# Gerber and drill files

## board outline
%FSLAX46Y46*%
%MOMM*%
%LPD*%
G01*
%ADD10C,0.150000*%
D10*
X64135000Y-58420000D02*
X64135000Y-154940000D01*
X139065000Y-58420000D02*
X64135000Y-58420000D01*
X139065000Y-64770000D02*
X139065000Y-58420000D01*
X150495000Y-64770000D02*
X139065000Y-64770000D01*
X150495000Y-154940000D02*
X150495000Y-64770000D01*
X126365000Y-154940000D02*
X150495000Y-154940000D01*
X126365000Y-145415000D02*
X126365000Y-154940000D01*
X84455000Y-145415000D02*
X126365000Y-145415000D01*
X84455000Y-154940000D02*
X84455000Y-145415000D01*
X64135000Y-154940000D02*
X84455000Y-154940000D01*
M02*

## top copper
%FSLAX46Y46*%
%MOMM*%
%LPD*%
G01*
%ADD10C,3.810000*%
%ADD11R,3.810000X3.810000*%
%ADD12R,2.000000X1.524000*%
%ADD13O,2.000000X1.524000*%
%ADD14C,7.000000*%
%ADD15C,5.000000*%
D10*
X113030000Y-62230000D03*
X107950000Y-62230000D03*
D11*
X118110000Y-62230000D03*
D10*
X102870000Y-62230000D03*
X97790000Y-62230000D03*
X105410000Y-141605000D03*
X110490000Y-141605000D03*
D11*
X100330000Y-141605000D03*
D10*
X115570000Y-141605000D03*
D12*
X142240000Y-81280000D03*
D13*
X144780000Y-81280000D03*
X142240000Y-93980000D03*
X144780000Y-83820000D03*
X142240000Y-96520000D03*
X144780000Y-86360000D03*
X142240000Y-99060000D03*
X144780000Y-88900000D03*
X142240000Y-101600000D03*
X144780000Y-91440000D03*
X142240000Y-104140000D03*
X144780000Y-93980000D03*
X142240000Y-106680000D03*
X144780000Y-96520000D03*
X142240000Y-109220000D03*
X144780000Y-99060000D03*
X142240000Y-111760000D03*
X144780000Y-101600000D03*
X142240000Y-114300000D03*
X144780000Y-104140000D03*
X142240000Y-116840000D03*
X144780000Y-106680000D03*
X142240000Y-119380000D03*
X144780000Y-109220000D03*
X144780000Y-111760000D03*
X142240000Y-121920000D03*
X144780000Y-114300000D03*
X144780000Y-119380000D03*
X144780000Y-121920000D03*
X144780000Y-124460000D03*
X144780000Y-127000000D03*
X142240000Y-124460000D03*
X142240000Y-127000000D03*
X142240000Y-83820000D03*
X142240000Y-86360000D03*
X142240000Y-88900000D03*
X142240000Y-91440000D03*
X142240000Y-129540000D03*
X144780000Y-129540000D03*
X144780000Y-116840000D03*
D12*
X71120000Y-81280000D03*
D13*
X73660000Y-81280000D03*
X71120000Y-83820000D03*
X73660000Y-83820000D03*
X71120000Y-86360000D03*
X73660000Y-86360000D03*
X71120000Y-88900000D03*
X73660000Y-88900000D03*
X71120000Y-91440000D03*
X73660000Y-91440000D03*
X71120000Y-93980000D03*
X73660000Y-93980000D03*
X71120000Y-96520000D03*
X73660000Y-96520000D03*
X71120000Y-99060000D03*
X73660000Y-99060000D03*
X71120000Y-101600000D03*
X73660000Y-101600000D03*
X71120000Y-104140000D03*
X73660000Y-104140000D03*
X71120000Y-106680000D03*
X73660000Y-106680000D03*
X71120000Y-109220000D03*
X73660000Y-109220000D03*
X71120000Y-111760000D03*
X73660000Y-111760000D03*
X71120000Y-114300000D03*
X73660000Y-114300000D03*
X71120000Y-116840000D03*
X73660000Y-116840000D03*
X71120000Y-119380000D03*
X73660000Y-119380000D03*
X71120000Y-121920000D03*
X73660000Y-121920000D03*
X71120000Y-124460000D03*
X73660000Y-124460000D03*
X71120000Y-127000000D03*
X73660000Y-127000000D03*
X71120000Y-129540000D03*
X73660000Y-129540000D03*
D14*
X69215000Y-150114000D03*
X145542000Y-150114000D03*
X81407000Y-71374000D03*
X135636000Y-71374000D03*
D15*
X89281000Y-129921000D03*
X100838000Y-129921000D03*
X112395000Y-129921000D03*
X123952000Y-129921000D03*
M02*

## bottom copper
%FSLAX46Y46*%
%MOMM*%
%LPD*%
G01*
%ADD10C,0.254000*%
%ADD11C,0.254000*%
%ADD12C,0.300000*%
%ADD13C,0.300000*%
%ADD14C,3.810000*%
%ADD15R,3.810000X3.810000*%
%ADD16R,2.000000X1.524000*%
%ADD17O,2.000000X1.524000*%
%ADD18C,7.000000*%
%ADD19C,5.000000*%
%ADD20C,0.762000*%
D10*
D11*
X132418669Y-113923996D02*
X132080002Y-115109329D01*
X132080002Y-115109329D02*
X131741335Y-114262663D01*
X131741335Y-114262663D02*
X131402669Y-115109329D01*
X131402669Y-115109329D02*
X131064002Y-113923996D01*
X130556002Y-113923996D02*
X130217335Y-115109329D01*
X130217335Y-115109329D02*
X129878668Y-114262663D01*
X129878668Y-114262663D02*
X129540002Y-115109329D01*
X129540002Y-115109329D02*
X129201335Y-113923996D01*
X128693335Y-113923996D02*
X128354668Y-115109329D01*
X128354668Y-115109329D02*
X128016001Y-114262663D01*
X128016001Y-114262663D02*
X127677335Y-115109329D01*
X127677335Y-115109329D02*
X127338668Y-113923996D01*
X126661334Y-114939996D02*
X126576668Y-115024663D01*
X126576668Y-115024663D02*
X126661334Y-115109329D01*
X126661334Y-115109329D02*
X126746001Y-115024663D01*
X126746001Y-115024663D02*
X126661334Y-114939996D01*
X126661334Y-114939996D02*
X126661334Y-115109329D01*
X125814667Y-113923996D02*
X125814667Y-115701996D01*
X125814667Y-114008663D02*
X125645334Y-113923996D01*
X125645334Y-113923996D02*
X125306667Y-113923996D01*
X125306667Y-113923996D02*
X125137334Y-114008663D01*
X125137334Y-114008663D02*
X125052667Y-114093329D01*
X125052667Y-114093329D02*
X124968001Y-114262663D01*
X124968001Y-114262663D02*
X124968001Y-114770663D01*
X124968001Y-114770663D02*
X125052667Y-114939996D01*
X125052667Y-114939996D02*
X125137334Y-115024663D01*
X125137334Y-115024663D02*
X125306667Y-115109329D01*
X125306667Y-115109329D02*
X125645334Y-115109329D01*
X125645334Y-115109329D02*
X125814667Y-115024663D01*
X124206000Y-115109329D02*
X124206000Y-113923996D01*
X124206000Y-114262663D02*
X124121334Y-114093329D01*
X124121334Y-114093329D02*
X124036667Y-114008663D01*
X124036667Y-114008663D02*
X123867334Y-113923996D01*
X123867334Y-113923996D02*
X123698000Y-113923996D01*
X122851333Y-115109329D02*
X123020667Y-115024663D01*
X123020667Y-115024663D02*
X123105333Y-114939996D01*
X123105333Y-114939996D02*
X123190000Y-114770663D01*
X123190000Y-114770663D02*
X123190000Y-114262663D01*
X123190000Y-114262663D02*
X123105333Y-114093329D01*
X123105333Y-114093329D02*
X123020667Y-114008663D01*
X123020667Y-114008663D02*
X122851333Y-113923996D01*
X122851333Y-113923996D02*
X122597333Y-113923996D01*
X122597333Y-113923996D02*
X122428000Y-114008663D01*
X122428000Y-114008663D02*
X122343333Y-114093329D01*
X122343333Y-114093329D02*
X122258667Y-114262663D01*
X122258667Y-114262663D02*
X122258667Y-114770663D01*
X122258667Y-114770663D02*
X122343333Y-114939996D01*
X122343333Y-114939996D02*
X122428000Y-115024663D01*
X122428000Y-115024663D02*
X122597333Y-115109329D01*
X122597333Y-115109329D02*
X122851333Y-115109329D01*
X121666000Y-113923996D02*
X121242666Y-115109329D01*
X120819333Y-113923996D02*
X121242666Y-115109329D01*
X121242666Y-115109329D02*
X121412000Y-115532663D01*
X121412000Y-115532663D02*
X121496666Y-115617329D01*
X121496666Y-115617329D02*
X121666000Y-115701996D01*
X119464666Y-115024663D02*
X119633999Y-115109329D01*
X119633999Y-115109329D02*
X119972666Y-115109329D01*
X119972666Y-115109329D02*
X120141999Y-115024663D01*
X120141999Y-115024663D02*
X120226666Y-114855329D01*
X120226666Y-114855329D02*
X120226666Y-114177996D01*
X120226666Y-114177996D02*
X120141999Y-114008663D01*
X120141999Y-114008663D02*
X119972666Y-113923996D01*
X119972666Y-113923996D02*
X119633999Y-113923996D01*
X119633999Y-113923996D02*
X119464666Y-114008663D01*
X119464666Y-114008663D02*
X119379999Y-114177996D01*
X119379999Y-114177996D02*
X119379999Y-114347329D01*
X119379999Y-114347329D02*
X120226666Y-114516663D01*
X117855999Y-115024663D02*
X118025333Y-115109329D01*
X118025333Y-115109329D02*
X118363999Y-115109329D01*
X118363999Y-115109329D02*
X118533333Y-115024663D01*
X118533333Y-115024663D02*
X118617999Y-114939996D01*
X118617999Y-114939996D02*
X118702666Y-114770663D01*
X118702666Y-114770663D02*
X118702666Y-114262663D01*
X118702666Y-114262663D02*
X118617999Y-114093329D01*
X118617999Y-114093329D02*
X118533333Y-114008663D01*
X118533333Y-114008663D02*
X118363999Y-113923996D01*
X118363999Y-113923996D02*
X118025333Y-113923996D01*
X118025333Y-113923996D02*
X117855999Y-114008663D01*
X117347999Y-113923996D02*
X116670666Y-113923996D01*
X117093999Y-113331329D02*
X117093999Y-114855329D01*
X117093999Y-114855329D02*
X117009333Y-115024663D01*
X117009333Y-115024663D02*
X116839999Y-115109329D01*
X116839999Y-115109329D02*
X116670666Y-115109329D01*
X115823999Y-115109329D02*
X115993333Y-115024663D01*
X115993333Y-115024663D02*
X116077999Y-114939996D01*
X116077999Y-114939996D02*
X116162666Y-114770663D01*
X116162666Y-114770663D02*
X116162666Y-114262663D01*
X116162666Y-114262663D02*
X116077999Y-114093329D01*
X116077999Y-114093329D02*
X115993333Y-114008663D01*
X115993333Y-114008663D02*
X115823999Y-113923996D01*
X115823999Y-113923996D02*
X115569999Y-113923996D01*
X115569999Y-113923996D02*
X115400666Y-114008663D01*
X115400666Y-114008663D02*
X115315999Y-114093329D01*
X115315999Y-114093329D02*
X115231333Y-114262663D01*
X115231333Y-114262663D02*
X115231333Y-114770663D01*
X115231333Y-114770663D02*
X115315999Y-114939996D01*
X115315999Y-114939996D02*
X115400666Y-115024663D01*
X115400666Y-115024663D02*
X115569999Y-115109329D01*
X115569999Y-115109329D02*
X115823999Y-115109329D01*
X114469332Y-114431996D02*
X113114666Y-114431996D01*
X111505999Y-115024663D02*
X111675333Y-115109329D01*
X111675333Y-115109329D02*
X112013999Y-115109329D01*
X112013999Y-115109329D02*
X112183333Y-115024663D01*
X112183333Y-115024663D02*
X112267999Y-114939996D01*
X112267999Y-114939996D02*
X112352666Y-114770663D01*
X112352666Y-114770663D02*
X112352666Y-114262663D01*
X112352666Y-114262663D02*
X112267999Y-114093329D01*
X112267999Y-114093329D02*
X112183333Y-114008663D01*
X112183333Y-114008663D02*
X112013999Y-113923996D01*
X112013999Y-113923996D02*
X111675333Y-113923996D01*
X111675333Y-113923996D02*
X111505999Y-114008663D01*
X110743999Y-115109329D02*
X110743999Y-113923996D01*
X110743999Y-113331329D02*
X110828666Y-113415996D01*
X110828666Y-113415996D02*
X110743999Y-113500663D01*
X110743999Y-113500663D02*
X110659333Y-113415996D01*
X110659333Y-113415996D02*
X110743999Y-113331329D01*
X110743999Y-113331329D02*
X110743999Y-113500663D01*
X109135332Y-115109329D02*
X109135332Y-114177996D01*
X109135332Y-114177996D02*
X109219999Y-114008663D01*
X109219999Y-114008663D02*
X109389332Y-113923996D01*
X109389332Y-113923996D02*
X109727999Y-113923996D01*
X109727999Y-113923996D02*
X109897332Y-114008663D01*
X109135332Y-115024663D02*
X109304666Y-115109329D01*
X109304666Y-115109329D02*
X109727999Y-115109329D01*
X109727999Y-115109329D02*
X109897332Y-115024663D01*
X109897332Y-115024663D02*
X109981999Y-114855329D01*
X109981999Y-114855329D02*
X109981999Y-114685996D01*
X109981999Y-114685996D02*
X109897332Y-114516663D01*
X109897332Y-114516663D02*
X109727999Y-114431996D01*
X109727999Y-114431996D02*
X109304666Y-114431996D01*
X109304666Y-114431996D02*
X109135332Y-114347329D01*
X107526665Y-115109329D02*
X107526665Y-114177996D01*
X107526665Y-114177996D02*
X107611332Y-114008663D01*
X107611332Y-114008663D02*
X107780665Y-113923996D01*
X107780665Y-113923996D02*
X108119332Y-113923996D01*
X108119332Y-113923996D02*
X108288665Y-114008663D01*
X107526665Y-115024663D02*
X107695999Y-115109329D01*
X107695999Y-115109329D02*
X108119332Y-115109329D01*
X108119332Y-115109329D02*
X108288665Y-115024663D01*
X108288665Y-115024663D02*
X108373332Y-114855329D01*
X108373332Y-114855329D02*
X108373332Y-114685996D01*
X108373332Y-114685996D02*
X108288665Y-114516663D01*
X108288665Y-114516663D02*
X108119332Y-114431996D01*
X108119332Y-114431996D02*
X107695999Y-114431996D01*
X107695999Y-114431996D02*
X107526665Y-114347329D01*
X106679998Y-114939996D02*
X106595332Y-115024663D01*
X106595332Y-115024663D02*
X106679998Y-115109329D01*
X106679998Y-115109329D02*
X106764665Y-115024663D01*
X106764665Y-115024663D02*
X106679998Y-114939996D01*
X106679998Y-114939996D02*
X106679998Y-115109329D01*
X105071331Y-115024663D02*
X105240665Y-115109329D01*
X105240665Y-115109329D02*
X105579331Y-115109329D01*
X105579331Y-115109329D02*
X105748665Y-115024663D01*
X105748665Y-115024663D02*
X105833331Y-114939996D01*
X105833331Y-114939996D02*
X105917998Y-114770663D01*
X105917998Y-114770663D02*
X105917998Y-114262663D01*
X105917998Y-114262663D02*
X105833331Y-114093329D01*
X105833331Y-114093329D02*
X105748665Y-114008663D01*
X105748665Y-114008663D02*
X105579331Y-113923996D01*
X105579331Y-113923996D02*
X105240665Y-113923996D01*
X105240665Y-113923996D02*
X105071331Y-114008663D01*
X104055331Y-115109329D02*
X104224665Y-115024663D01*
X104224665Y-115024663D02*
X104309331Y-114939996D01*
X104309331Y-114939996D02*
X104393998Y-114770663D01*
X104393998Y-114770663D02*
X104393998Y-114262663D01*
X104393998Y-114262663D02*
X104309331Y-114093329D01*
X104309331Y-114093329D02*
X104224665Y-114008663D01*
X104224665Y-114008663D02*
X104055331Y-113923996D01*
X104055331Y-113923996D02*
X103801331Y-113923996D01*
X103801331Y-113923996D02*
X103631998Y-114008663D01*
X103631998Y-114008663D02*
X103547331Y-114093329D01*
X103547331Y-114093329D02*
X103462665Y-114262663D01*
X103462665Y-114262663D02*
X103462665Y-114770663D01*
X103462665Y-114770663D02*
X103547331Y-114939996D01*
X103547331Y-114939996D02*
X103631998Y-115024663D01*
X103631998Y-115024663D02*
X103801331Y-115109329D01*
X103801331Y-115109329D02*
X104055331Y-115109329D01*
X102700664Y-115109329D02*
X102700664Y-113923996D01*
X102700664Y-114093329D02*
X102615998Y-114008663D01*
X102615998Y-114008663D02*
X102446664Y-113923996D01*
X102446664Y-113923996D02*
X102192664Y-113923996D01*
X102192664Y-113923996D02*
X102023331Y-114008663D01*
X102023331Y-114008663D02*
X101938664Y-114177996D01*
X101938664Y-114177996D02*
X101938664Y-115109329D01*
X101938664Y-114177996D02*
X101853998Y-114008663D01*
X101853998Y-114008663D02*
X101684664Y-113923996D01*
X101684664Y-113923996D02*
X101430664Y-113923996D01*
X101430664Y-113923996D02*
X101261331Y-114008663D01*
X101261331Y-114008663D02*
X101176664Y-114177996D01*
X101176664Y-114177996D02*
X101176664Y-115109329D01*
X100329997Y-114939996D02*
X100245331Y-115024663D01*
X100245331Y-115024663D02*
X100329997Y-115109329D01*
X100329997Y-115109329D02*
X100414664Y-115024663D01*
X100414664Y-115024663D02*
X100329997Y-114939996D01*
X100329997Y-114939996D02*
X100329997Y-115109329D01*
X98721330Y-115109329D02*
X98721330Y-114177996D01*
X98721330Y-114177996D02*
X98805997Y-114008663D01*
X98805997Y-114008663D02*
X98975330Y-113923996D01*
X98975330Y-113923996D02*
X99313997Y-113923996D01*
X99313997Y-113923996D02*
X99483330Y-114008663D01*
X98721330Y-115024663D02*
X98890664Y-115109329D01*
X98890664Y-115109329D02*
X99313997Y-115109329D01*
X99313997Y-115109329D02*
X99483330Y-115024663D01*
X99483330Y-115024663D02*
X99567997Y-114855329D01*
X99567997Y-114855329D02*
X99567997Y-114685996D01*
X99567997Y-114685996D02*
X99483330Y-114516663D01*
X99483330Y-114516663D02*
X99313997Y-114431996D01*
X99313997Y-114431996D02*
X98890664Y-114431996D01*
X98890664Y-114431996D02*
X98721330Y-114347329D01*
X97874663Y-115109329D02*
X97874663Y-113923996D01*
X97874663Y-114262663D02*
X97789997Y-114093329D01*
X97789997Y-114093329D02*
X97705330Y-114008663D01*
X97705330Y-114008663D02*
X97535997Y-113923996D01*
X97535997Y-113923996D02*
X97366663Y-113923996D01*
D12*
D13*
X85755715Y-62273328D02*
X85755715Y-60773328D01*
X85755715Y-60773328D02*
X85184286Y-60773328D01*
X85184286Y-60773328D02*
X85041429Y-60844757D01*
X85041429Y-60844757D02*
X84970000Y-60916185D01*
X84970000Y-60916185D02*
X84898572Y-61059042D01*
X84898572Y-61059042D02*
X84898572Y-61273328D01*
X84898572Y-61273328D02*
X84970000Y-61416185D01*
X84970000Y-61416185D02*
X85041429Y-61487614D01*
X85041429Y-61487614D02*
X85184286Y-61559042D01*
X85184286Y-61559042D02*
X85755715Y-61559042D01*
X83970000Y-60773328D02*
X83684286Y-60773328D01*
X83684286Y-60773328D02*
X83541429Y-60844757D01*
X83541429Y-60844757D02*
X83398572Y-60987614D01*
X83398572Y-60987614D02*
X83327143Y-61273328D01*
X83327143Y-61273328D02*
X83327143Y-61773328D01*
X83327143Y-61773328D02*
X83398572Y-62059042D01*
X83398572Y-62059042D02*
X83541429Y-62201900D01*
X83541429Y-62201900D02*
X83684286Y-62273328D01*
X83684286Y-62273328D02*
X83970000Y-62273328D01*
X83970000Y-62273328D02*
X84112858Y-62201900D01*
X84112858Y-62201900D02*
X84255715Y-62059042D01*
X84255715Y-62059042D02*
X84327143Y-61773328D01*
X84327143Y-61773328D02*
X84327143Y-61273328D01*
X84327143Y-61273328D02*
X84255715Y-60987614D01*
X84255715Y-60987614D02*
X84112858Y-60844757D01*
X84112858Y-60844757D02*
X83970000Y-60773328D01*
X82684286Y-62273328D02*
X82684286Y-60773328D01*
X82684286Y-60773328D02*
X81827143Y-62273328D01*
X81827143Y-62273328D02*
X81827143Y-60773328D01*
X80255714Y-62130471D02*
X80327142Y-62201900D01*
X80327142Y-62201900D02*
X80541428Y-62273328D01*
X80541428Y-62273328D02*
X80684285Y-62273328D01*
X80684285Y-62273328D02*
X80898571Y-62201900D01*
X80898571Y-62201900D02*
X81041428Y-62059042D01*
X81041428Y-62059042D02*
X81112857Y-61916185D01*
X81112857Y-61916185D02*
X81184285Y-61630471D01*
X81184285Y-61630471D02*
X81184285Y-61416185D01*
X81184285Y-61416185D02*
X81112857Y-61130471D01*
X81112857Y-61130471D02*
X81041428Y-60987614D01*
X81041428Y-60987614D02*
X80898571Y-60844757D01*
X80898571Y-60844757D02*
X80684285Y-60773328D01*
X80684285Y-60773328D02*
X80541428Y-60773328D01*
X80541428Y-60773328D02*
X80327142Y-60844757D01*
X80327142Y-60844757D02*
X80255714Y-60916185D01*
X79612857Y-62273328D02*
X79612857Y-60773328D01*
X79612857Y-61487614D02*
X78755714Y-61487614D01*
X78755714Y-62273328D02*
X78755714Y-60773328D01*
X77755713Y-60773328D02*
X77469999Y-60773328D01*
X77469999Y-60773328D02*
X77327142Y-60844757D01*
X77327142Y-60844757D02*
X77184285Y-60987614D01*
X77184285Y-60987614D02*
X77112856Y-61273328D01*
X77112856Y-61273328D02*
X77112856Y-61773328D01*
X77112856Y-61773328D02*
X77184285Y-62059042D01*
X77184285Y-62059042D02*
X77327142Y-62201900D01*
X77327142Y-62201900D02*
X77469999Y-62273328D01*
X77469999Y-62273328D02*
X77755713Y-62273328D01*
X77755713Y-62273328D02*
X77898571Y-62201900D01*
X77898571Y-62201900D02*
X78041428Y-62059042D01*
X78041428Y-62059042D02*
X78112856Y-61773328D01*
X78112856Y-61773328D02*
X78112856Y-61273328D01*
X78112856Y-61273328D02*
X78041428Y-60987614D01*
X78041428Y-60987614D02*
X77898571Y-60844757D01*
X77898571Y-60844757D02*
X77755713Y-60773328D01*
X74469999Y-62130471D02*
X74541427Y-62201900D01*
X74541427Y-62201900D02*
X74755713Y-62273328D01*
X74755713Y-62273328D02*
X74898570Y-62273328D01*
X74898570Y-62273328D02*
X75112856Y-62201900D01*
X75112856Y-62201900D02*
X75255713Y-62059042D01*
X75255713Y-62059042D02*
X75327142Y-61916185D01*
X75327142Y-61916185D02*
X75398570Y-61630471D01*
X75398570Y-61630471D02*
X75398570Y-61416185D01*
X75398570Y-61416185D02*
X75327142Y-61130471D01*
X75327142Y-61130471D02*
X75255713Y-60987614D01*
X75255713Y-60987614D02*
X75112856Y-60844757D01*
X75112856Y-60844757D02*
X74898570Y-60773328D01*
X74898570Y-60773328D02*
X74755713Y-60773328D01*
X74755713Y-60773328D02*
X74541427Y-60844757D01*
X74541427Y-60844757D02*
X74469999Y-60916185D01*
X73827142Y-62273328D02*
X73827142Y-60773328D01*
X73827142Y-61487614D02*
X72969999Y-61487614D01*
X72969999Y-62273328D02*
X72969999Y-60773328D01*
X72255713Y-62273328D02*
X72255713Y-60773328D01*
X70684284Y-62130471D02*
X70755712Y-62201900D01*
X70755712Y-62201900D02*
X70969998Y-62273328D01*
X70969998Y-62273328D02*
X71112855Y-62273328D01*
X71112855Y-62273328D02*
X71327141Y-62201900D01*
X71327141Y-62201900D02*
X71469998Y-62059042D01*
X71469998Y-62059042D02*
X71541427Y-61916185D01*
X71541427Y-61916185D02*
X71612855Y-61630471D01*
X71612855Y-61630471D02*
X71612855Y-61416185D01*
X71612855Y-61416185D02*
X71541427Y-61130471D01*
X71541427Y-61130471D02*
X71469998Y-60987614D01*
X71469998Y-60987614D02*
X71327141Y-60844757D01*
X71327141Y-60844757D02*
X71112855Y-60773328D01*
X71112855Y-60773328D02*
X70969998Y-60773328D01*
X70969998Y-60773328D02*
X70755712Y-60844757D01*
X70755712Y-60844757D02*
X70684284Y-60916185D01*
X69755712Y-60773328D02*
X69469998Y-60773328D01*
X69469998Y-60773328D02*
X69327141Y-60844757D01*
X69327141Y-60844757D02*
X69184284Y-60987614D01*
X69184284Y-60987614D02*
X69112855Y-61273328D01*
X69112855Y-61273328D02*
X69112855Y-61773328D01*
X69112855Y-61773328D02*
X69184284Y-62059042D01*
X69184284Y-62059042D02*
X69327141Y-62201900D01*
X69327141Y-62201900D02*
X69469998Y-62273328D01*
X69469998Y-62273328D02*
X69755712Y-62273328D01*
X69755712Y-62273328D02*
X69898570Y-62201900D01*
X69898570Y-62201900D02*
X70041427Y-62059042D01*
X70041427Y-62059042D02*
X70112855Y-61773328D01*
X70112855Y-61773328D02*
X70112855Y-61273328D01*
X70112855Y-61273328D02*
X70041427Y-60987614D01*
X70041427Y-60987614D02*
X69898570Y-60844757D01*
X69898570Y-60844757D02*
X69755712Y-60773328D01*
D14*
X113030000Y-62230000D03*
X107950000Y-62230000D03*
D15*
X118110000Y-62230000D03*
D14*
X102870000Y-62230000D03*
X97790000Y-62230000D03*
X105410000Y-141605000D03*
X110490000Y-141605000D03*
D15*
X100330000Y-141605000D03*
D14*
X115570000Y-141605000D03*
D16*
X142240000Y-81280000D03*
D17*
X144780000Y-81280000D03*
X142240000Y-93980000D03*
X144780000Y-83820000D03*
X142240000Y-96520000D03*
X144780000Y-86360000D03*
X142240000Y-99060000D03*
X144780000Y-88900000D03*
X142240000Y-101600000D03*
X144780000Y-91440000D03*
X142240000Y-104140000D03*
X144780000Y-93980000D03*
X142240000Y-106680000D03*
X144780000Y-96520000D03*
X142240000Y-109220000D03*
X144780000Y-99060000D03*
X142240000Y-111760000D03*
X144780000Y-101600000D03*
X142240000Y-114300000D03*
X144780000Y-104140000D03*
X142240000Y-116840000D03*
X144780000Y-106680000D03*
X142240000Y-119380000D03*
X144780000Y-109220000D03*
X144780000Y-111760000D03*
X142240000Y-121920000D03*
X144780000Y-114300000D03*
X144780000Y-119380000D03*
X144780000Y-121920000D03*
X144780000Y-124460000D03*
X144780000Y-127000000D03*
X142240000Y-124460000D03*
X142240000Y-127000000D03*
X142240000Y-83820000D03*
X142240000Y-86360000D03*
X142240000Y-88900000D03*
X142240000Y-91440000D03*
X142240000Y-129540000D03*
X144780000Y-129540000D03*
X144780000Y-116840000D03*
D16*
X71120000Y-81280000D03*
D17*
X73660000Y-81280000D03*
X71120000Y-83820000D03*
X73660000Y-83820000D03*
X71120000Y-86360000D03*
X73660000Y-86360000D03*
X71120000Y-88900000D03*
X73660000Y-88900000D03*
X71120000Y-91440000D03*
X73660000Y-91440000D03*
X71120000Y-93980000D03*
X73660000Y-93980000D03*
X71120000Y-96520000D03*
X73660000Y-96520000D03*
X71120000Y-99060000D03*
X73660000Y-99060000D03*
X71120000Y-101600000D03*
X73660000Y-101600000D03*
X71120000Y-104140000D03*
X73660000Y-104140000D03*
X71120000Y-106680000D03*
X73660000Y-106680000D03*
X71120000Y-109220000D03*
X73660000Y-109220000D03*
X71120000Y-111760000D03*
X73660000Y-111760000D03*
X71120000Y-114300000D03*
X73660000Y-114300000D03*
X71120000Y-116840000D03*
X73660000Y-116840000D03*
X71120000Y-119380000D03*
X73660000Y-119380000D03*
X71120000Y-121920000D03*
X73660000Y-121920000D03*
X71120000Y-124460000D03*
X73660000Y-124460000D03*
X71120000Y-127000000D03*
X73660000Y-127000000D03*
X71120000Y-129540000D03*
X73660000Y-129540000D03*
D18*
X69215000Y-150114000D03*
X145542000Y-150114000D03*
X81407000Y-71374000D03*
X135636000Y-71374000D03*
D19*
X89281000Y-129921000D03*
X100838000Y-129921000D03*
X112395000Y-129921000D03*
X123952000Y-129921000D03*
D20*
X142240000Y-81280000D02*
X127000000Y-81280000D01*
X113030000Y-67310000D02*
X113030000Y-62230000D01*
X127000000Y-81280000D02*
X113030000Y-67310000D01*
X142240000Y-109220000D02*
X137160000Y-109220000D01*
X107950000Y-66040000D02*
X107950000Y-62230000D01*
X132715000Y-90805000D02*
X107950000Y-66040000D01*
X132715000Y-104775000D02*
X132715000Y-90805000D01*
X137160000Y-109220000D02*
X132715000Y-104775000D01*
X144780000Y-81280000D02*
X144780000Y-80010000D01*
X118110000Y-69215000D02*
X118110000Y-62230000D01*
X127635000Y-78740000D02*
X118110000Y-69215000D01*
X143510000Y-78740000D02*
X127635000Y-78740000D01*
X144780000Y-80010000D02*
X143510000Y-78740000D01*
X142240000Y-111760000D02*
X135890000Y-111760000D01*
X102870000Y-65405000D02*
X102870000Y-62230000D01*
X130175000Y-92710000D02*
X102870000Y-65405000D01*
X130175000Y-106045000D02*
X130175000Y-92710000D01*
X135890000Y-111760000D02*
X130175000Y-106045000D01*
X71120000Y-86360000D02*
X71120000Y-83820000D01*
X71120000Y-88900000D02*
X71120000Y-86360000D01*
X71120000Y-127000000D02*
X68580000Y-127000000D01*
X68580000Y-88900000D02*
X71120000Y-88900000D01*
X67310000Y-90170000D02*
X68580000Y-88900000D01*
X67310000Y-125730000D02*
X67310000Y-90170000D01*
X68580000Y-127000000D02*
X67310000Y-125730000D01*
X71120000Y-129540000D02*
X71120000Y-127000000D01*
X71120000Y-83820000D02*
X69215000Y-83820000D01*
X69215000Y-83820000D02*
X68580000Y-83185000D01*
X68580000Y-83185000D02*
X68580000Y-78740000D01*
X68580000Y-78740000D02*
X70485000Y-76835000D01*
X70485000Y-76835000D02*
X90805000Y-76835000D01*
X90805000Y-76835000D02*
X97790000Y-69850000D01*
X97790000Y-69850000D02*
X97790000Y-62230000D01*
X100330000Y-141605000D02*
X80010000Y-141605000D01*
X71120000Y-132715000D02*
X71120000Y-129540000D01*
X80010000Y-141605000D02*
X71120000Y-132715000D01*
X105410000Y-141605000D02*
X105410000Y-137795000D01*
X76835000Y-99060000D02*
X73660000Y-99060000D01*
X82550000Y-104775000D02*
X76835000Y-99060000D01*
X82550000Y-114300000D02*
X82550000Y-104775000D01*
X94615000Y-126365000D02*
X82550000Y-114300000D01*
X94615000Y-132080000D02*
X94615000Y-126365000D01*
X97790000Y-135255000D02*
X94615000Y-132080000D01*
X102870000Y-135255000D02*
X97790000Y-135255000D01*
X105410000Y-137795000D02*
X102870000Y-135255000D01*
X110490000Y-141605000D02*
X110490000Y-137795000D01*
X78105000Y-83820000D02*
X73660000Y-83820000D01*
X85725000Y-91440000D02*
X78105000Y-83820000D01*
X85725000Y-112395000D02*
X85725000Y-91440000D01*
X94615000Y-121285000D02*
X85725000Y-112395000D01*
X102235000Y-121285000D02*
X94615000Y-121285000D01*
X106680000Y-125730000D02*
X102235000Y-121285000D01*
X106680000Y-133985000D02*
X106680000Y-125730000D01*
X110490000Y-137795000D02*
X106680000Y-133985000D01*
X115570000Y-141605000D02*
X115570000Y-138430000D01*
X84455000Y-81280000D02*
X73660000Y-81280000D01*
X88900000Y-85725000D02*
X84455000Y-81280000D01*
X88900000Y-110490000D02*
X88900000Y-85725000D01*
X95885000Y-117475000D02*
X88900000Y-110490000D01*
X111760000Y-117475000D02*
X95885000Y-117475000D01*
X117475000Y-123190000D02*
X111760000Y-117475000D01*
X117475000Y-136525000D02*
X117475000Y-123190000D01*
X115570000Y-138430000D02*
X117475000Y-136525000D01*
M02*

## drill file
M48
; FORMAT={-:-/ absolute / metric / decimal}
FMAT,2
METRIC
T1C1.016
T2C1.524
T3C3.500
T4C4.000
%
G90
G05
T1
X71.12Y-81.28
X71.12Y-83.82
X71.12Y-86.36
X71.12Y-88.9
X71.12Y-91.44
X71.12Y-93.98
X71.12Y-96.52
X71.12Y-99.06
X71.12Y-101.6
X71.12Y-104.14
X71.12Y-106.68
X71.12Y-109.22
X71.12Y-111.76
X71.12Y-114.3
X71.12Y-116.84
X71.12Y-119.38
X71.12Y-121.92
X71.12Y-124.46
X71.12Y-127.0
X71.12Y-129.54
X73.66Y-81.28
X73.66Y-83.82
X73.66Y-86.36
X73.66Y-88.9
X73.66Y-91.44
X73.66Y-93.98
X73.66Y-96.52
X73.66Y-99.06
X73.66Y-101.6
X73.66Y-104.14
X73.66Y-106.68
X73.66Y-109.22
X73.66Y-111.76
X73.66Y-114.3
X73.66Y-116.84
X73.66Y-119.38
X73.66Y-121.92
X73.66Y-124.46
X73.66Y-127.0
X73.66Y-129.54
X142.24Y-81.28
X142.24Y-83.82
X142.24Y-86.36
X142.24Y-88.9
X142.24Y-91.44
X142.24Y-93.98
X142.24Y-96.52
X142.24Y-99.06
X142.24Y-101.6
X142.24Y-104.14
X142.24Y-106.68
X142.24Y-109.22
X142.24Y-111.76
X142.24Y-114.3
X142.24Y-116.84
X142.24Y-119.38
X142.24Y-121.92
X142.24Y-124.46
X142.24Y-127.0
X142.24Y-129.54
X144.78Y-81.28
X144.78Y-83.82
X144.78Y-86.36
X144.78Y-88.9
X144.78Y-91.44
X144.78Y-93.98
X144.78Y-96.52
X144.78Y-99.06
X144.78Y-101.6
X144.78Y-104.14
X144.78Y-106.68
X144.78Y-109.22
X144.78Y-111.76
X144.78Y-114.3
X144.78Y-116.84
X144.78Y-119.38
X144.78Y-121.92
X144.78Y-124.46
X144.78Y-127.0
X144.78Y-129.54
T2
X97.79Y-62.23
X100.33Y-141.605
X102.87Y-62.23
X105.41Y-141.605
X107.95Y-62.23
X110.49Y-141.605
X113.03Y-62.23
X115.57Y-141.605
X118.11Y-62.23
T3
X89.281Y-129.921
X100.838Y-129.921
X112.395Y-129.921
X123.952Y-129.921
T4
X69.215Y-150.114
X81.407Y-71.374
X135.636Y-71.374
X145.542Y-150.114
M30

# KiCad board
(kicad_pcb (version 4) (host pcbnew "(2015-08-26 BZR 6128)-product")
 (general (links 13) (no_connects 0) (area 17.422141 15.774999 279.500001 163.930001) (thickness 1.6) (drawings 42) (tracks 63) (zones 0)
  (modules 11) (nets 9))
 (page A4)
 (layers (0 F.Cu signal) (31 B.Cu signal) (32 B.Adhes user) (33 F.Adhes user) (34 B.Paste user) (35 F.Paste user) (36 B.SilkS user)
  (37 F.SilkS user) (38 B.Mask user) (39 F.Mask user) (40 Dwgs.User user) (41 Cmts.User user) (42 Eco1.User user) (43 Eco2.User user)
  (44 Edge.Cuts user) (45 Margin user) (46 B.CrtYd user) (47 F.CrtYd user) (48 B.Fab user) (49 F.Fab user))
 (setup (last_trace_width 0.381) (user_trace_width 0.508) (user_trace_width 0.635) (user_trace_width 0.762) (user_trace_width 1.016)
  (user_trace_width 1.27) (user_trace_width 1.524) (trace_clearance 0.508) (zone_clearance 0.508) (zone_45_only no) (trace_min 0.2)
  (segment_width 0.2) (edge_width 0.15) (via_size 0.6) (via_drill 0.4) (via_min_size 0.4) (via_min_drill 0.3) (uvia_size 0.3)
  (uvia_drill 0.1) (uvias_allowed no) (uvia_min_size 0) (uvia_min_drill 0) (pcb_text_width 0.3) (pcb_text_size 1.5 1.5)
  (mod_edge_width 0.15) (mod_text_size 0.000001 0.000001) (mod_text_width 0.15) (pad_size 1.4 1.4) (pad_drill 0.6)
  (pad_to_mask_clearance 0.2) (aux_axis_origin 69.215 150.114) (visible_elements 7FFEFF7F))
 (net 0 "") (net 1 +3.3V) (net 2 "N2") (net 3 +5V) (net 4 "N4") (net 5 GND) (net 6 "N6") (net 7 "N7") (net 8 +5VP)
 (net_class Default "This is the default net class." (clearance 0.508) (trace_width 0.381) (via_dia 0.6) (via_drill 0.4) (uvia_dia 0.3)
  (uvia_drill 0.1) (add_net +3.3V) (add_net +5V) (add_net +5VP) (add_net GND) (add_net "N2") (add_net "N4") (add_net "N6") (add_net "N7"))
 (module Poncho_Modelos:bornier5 (layer F.Cu) (at 107.95 62.23 180)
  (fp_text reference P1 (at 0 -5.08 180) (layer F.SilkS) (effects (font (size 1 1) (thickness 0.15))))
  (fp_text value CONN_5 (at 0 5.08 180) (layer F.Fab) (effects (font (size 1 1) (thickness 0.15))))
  (pad 2 thru_hole circle (at -5.08 0 180) (size 3.81 3.81) (drill 1.524) (layers *.Cu *.Mask F.SilkS) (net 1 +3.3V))
  (pad 3 thru_hole circle (at 0 0 180) (size 3.81 3.81) (drill 1.524) (layers *.Cu *.Mask F.SilkS) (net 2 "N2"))
  (pad 1 thru_hole rect (at -10.16 0 180) (size 3.81 3.81) (drill 1.524) (layers *.Cu *.Mask F.SilkS) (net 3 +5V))
  (pad 4 thru_hole circle (at 5.08 0 180) (size 3.81 3.81) (drill 1.524) (layers *.Cu *.Mask F.SilkS) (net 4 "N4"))
  (pad 5 thru_hole circle (at 10.16 0 180) (size 3.81 3.81) (drill 1.524) (layers *.Cu *.Mask F.SilkS) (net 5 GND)))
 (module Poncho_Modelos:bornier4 (layer F.Cu) (at 107.95 141.605)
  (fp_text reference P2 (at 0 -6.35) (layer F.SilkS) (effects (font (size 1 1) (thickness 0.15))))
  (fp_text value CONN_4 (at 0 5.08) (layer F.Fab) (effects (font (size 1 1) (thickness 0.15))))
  (pad 2 thru_hole circle (at -2.54 0) (size 3.81 3.81) (drill 1.524) (layers *.Cu *.Mask F.SilkS) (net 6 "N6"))
  (pad 3 thru_hole circle (at 2.54 0) (size 3.81 3.81) (drill 1.524) (layers *.Cu *.Mask F.SilkS) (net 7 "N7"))
  (pad 1 thru_hole rect (at -7.62 0) (size 3.81 3.81) (drill 1.524) (layers *.Cu *.Mask F.SilkS) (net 5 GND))
  (pad 4 thru_hole circle (at 7.62 0) (size 3.81 3.81) (drill 1.524) (layers *.Cu *.Mask F.SilkS) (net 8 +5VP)))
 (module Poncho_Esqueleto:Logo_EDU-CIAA (layer F.Cu) (at 120.65 100.965)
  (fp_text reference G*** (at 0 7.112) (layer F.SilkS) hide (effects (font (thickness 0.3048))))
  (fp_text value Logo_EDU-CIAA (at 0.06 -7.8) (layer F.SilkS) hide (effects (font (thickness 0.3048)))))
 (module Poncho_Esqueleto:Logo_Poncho (layer F.Cu) (at 96.52 100.965)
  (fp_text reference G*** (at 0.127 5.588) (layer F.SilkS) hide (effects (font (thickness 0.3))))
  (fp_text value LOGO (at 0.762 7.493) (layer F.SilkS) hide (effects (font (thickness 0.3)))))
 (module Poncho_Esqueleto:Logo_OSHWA (layer F.Cu) (at 107.315 100.965)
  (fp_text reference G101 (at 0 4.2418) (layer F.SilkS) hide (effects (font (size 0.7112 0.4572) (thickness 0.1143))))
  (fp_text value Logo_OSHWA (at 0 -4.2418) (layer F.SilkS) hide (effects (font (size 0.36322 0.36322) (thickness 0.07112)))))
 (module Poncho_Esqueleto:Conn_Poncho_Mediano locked (layer F.Cu) (at 142.24 81.28)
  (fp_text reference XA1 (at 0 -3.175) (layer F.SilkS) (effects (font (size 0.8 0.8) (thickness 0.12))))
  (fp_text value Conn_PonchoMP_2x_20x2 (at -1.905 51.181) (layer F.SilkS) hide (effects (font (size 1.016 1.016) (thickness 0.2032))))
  (pad 1 thru_hole rect (at 0 0 270) (size 1.524 2) (drill 1.016) (layers *.Cu *.Mask F.SilkS) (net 1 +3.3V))
  (pad 2 thru_hole oval (at 2.54 0 270) (size 1.524 2) (drill 1.016) (layers *.Cu *.Mask F.SilkS) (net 3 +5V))
  (pad 11 thru_hole oval (at 0 12.7 270) (size 1.524 2) (drill 1.016) (layers *.Cu *.Mask F.SilkS))
  (pad 4 thru_hole oval (at 2.54 2.54 270) (size 1.524 2) (drill 1.016) (layers *.Cu *.Mask F.SilkS))
  (pad 13 thru_hole oval (at 0 15.24 270) (size 1.524 2) (drill 1.016) (layers *.Cu *.Mask F.SilkS))
  (pad 6 thru_hole oval (at 2.54 5.08 270) (size 1.524 2) (drill 1.016) (layers *.Cu *.Mask F.SilkS))
  (pad 15 thru_hole oval (at 0 17.78 270) (size 1.524 2) (drill 1.016) (layers *.Cu *.Mask F.SilkS))
  (pad 8 thru_hole oval (at 2.54 7.62 270) (size 1.524 2) (drill 1.016) (layers *.Cu *.Mask F.SilkS))
  (pad 17 thru_hole oval (at 0 20.32 270) (size 1.524 2) (drill 1.016) (layers *.Cu *.Mask F.SilkS))
  (pad 10 thru_hole oval (at 2.54 10.16 270) (size 1.524 2) (drill 1.016) (layers *.Cu *.Mask F.SilkS))
  (pad 19 thru_hole oval (at 0 22.86 270) (size 1.524 2) (drill 1.016) (layers *.Cu *.Mask F.SilkS))
  (pad 12 thru_hole oval (at 2.54 12.7 270) (size 1.524 2) (drill 1.016) (layers *.Cu *.Mask F.SilkS))
  (pad 21 thru_hole oval (at 0 25.4 270) (size 1.524 2) (drill 1.016) (layers *.Cu *.Mask F.SilkS))
  (pad 14 thru_hole oval (at 2.54 15.24 270) (size 1.524 2) (drill 1.016) (layers *.Cu *.Mask F.SilkS))
  (pad 23 thru_hole oval (at 0 27.94 270) (size 1.524 2) (drill 1.016) (layers *.Cu *.Mask F.SilkS) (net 2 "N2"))
  (pad 16 thru_hole oval (at 2.54 17.78 270) (size 1.524 2) (drill 1.016) (layers *.Cu *.Mask F.SilkS))
  (pad 25 thru_hole oval (at 0 30.48 270) (size 1.524 2) (drill 1.016) (layers *.Cu *.Mask F.SilkS) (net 4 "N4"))
  (pad 18 thru_hole oval (at 2.54 20.32 270) (size 1.524 2) (drill 1.016) (layers *.Cu *.Mask F.SilkS))
  (pad 27 thru_hole oval (at 0 33.02 270) (size 1.524 2) (drill 1.016) (layers *.Cu *.Mask F.SilkS))
  (pad 20 thru_hole oval (at 2.54 22.86 270) (size 1.524 2) (drill 1.016) (layers *.Cu *.Mask F.SilkS))
  (pad 29 thru_hole oval (at 0 35.56 270) (size 1.524 2) (drill 1.016) (layers *.Cu *.Mask F.SilkS))
  (pad 22 thru_hole oval (at 2.54 25.4 270) (size 1.524 2) (drill 1.016) (layers *.Cu *.Mask F.SilkS))
  (pad 31 thru_hole oval (at 0 38.1 270) (size 1.524 2) (drill 1.016) (layers *.Cu *.Mask F.SilkS))
  (pad 24 thru_hole oval (at 2.54 27.94 270) (size 1.524 2) (drill 1.016) (layers *.Cu *.Mask F.SilkS))
  (pad 26 thru_hole oval (at 2.54 30.48 270) (size 1.524 2) (drill 1.016) (layers *.Cu *.Mask F.SilkS))
  (pad 33 thru_hole oval (at 0 40.64 270) (size 1.524 2) (drill 1.016) (layers *.Cu *.Mask F.SilkS))
  (pad 28 thru_hole oval (at 2.54 33.02 270) (size 1.524 2) (drill 1.016) (layers *.Cu *.Mask F.SilkS))
  (pad 32 thru_hole oval (at 2.54 38.1 270) (size 1.524 2) (drill 1.016) (layers *.Cu *.Mask F.SilkS))
  (pad 34 thru_hole oval (at 2.54 40.64 270) (size 1.524 2) (drill 1.016) (layers *.Cu *.Mask F.SilkS))
  (pad 36 thru_hole oval (at 2.54 43.18 270) (size 1.524 2) (drill 1.016) (layers *.Cu *.Mask F.SilkS))
  (pad 38 thru_hole oval (at 2.54 45.72 270) (size 1.524 2) (drill 1.016) (layers *.Cu *.Mask F.SilkS))
  (pad 35 thru_hole oval (at 0 43.18 270) (size 1.524 2) (drill 1.016) (layers *.Cu *.Mask F.SilkS))
  (pad 37 thru_hole oval (at 0 45.72 270) (size 1.524 2) (drill 1.016) (layers *.Cu *.Mask F.SilkS))
  (pad 3 thru_hole oval (at 0 2.54 270) (size 1.524 2) (drill 1.016) (layers *.Cu *.Mask F.SilkS))
  (pad 5 thru_hole oval (at 0 5.08 270) (size 1.524 2) (drill 1.016) (layers *.Cu *.Mask F.SilkS))
  (pad 7 thru_hole oval (at 0 7.62 270) (size 1.524 2) (drill 1.016) (layers *.Cu *.Mask F.SilkS))
  (pad 9 thru_hole oval (at 0 10.16 270) (size 1.524 2) (drill 1.016) (layers *.Cu *.Mask F.SilkS))
  (pad 39 thru_hole oval (at 0 48.26 270) (size 1.524 2) (drill 1.016) (layers *.Cu *.Mask F.SilkS))
  (pad 40 thru_hole oval (at 2.54 48.26 270) (size 1.524 2) (drill 1.016) (layers *.Cu *.Mask F.SilkS))
  (pad 30 thru_hole oval (at 2.54 35.56 270) (size 1.524 2) (drill 1.016) (layers *.Cu *.Mask F.SilkS))
  (pad 41 thru_hole rect (at -71.12 0 270) (size 1.524 2) (drill 1.016) (layers *.Cu *.Mask F.SilkS))
  (pad 42 thru_hole oval (at -68.58 0 270) (size 1.524 2) (drill 1.016) (layers *.Cu *.Mask F.SilkS) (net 8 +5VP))
  (pad 43 thru_hole oval (at -71.12 2.54 270) (size 1.524 2) (drill 1.016) (layers *.Cu *.Mask F.SilkS) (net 5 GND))
  (pad 44 thru_hole oval (at -68.58 2.54 270) (size 1.524 2) (drill 1.016) (layers *.Cu *.Mask F.SilkS) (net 7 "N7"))
  (pad 45 thru_hole oval (at -71.12 5.08 270) (size 1.524 2) (drill 1.016) (layers *.Cu *.Mask F.SilkS) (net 5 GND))
  (pad 46 thru_hole oval (at -68.58 5.08 270) (size 1.524 2) (drill 1.016) (layers *.Cu *.Mask F.SilkS))
  (pad 47 thru_hole oval (at -71.12 7.62 270) (size 1.524 2) (drill 1.016) (layers *.Cu *.Mask F.SilkS) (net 5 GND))
  (pad 48 thru_hole oval (at -68.58 7.62 270) (size 1.524 2) (drill 1.016) (layers *.Cu *.Mask F.SilkS))
  (pad 49 thru_hole oval (at -71.12 10.16 270) (size 1.524 2) (drill 1.016) (layers *.Cu *.Mask F.SilkS))
  (pad 50 thru_hole oval (at -68.58 10.16 270) (size 1.524 2) (drill 1.016) (layers *.Cu *.Mask F.SilkS))
  (pad 51 thru_hole oval (at -71.12 12.7 270) (size 1.524 2) (drill 1.016) (layers *.Cu *.Mask F.SilkS))
  (pad 52 thru_hole oval (at -68.58 12.7 270) (size 1.524 2) (drill 1.016) (layers *.Cu *.Mask F.SilkS))
  (pad 53 thru_hole oval (at -71.12 15.24 270) (size 1.524 2) (drill 1.016) (layers *.Cu *.Mask F.SilkS))
  (pad 54 thru_hole oval (at -68.58 15.24 270) (size 1.524 2) (drill 1.016) (layers *.Cu *.Mask F.SilkS))
  (pad 55 thru_hole oval (at -71.12 17.78 270) (size 1.524 2) (drill 1.016) (layers *.Cu *.Mask F.SilkS))
  (pad 56 thru_hole oval (at -68.58 17.78 270) (size 1.524 2) (drill 1.016) (layers *.Cu *.Mask F.SilkS) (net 6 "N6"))
  (pad 57 thru_hole oval (at -71.12 20.32 270) (size 1.524 2) (drill 1.016) (layers *.Cu *.Mask F.SilkS))
  (pad 58 thru_hole oval (at -68.58 20.32 270) (size 1.524 2) (drill 1.016) (layers *.Cu *.Mask F.SilkS))
  (pad 59 thru_hole oval (at -71.12 22.86 270) (size 1.524 2) (drill 1.016) (layers *.Cu *.Mask F.SilkS))
  (pad 60 thru_hole oval (at -68.58 22.86 270) (size 1.524 2) (drill 1.016) (layers *.Cu *.Mask F.SilkS))
  (pad 61 thru_hole oval (at -71.12 25.4 270) (size 1.524 2) (drill 1.016) (layers *.Cu *.Mask F.SilkS))
  (pad 62 thru_hole oval (at -68.58 25.4 270) (size 1.524 2) (drill 1.016) (layers *.Cu *.Mask F.SilkS))
  (pad 63 thru_hole oval (at -71.12 27.94 270) (size 1.524 2) (drill 1.016) (layers *.Cu *.Mask F.SilkS))
  (pad 64 thru_hole oval (at -68.58 27.94 270) (size 1.524 2) (drill 1.016) (layers *.Cu *.Mask F.SilkS))
  (pad 65 thru_hole oval (at -71.12 30.48 270) (size 1.524 2) (drill 1.016) (layers *.Cu *.Mask F.SilkS))
  (pad 66 thru_hole oval (at -68.58 30.48 270) (size 1.524 2) (drill 1.016) (layers *.Cu *.Mask F.SilkS))
  (pad 67 thru_hole oval (at -71.12 33.02 270) (size 1.524 2) (drill 1.016) (layers *.Cu *.Mask F.SilkS))
  (pad 68 thru_hole oval (at -68.58 33.02 270) (size 1.524 2) (drill 1.016) (layers *.Cu *.Mask F.SilkS))
  (pad 69 thru_hole oval (at -71.12 35.56 270) (size 1.524 2) (drill 1.016) (layers *.Cu *.Mask F.SilkS))
  (pad 70 thru_hole oval (at -68.58 35.56 270) (size 1.524 2) (drill 1.016) (layers *.Cu *.Mask F.SilkS))
  (pad 71 thru_hole oval (at -71.12 38.1 270) (size 1.524 2) (drill 1.016) (layers *.Cu *.Mask F.SilkS))
  (pad 72 thru_hole oval (at -68.58 38.1 270) (size 1.524 2) (drill 1.016) (layers *.Cu *.Mask F.SilkS))
  (pad 73 thru_hole oval (at -71.12 40.64 270) (size 1.524 2) (drill 1.016) (layers *.Cu *.Mask F.SilkS))
  (pad 74 thru_hole oval (at -68.58 40.64 270) (size 1.524 2) (drill 1.016) (layers *.Cu *.Mask F.SilkS))
  (pad 75 thru_hole oval (at -71.12 43.18 270) (size 1.524 2) (drill 1.016) (layers *.Cu *.Mask F.SilkS))
  (pad 76 thru_hole oval (at -68.58 43.18 270) (size 1.524 2) (drill 1.016) (layers *.Cu *.Mask F.SilkS))
  (pad 77 thru_hole oval (at -71.12 45.72 270) (size 1.524 2) (drill 1.016) (layers *.Cu *.Mask F.SilkS) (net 5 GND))
  (pad 78 thru_hole oval (at -68.58 45.72 270) (size 1.524 2) (drill 1.016) (layers *.Cu *.Mask F.SilkS))
  (pad 79 thru_hole oval (at -71.12 48.26 270) (size 1.524 2) (drill 1.016) (layers *.Cu *.Mask F.SilkS) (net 5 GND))
  (pad 80 thru_hole oval (at -68.58 48.26 270) (size 1.524 2) (drill 1.016) (layers *.Cu *.Mask F.SilkS))
  (pad ~ thru_hole circle (at -73.025 68.834) (size 7 7) (drill 4) (layers *.Cu *.Mask F.SilkS))
  (pad ~ thru_hole circle (at 3.302 68.834) (size 7 7) (drill 4) (layers *.Cu *.Mask F.SilkS))
  (pad ~ thru_hole circle (at -60.833 -9.906) (size 7 7) (drill 4) (layers *.Cu *.Mask F.SilkS))
  (pad ~ thru_hole circle (at -6.604 -9.906) (size 7 7) (drill 4) (layers *.Cu *.Mask F.SilkS)))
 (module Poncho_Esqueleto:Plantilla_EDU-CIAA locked (layer F.Cu) (at 142.24 81.28)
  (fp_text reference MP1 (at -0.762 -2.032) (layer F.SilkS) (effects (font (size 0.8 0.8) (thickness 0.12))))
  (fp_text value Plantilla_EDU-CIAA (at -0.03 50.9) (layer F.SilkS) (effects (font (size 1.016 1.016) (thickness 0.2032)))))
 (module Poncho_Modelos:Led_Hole (layer F.Cu) (at 89.281 129.921)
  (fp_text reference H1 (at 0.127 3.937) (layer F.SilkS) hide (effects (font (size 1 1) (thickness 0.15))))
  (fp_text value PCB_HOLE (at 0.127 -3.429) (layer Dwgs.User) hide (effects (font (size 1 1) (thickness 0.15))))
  (pad 1 thru_hole circle (at 0 0) (size 5 5) (drill 3.5) (layers *.Cu *.Mask F.SilkS)))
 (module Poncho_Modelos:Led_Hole (layer F.Cu) (at 100.838 129.921)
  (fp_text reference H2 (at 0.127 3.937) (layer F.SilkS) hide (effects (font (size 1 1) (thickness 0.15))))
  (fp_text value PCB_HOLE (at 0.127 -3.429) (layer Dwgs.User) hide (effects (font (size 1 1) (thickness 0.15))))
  (pad 1 thru_hole circle (at 0 0) (size 5 5) (drill 3.5) (layers *.Cu *.Mask F.SilkS)))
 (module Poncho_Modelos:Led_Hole (layer F.Cu) (at 112.395 129.921)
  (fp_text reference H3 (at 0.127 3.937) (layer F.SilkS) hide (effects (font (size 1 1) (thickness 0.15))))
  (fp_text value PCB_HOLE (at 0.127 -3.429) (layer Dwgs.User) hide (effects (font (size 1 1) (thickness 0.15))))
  (pad 1 thru_hole circle (at 0 0) (size 5 5) (drill 3.5) (layers *.Cu *.Mask F.SilkS)))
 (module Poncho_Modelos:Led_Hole (layer F.Cu) (at 123.952 129.921)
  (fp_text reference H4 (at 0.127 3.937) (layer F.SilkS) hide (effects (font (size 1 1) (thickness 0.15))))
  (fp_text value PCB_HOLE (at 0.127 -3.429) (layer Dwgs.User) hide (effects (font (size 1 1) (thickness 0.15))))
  (pad 1 thru_hole circle (at 0 0) (size 5 5) (drill 3.5) (layers *.Cu *.Mask F.SilkS)))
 (gr_line (start 64.135 58.42) (end 64.135 154.94) (angle 90) (layer Edge.Cuts) (width 0.15))
 (gr_line (start 139.065 58.42) (end 64.135 58.42) (angle 90) (layer Edge.Cuts) (width 0.15))
 (gr_line (start 139.065 64.77) (end 139.065 58.42) (angle 90) (layer Edge.Cuts) (width 0.15))
 (gr_line (start 150.495 64.77) (end 139.065 64.77) (angle 90) (layer Edge.Cuts) (width 0.15))
 (gr_line (start 150.495 154.94) (end 150.495 64.77) (angle 90) (layer Edge.Cuts) (width 0.15))
 (gr_line (start 126.365 154.94) (end 150.495 154.94) (angle 90) (layer Edge.Cuts) (width 0.15))
 (gr_line (start 126.365 145.415) (end 126.365 154.94) (angle 90) (layer Edge.Cuts) (width 0.15))
 (gr_line (start 84.455 145.415) (end 126.365 145.415) (angle 90) (layer Edge.Cuts) (width 0.15))
 (gr_line (start 84.455 154.94) (end 84.455 145.415) (angle 90) (layer Edge.Cuts) (width 0.15))
 (gr_line (start 64.135 154.94) (end 84.455 154.94) (angle 90) (layer Edge.Cuts) (width 0.15))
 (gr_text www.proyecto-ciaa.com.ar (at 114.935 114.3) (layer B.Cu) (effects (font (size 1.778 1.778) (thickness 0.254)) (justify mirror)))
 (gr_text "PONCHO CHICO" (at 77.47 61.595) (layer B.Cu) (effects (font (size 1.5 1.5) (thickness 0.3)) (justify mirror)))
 (segment (start 142.24 81.28) (end 127 81.28) (width 0.762) (layer B.Cu) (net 1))
 (segment (start 113.03 67.31) (end 113.03 62.23) (width 0.762) (layer B.Cu) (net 1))
 (segment (start 127 81.28) (end 113.03 67.31) (width 0.762) (layer B.Cu) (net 1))
 (segment (start 142.24 109.22) (end 137.16 109.22) (width 0.762) (layer B.Cu) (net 2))
 (segment (start 107.95 66.04) (end 107.95 62.23) (width 0.762) (layer B.Cu) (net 2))
 (segment (start 132.715 90.805) (end 107.95 66.04) (width 0.762) (layer B.Cu) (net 2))
 (segment (start 132.715 104.775) (end 132.715 90.805) (width 0.762) (layer B.Cu) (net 2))
 (segment (start 137.16 109.22) (end 132.715 104.775) (width 0.762) (layer B.Cu) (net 2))
 (segment (start 144.78 81.28) (end 144.78 80.01) (width 0.762) (layer B.Cu) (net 3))
 (segment (start 118.11 69.215) (end 118.11 62.23) (width 0.762) (layer B.Cu) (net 3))
 (segment (start 127.635 78.74) (end 118.11 69.215) (width 0.762) (layer B.Cu) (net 3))
 (segment (start 143.51 78.74) (end 127.635 78.74) (width 0.762) (layer B.Cu) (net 3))
 (segment (start 144.78 80.01) (end 143.51 78.74) (width 0.762) (layer B.Cu) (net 3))
 (segment (start 142.24 111.76) (end 135.89 111.76) (width 0.762) (layer B.Cu) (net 4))
 (segment (start 102.87 65.405) (end 102.87 62.23) (width 0.762) (layer B.Cu) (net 4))
 (segment (start 130.175 92.71) (end 102.87 65.405) (width 0.762) (layer B.Cu) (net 4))
 (segment (start 130.175 106.045) (end 130.175 92.71) (width 0.762) (layer B.Cu) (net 4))
 (segment (start 135.89 111.76) (end 130.175 106.045) (width 0.762) (layer B.Cu) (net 4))
 (segment (start 71.12 86.36) (end 71.12 83.82) (width 0.762) (layer B.Cu) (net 5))
 (segment (start 71.12 88.9) (end 71.12 86.36) (width 0.762) (layer B.Cu) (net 5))
 (segment (start 71.12 127) (end 68.58 127) (width 0.762) (layer B.Cu) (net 5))
 (segment (start 68.58 88.9) (end 71.12 88.9) (width 0.762) (layer B.Cu) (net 5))
 (segment (start 67.31 90.17) (end 68.58 88.9) (width 0.762) (layer B.Cu) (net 5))
 (segment (start 67.31 125.73) (end 67.31 90.17) (width 0.762) (layer B.Cu) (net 5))
 (segment (start 68.58 127) (end 67.31 125.73) (width 0.762) (layer B.Cu) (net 5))
 (segment (start 71.12 129.54) (end 71.12 127) (width 0.762) (layer B.Cu) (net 5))
 (segment (start 71.12 83.82) (end 69.215 83.82) (width 0.762) (layer B.Cu) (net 5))
 (segment (start 69.215 83.82) (end 68.58 83.185) (width 0.762) (layer B.Cu) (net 5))
 (segment (start 68.58 83.185) (end 68.58 78.74) (width 0.762) (layer B.Cu) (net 5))
 (segment (start 68.58 78.74) (end 70.485 76.835) (width 0.762) (layer B.Cu) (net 5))
 (segment (start 70.485 76.835) (end 90.805 76.835) (width 0.762) (layer B.Cu) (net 5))
 (segment (start 90.805 76.835) (end 97.79 69.85) (width 0.762) (layer B.Cu) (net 5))
 (segment (start 97.79 69.85) (end 97.79 62.23) (width 0.762) (layer B.Cu) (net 5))
 (segment (start 100.33 141.605) (end 80.01 141.605) (width 0.762) (layer B.Cu) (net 5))
 (segment (start 71.12 132.715) (end 71.12 129.54) (width 0.762) (layer B.Cu) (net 5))
 (segment (start 80.01 141.605) (end 71.12 132.715) (width 0.762) (layer B.Cu) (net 5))
 (segment (start 105.41 141.605) (end 105.41 137.795) (width 0.762) (layer B.Cu) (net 6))
 (segment (start 76.835 99.06) (end 73.66 99.06) (width 0.762) (layer B.Cu) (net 6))
 (segment (start 82.55 104.775) (end 76.835 99.06) (width 0.762) (layer B.Cu) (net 6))
 (segment (start 82.55 114.3) (end 82.55 104.775) (width 0.762) (layer B.Cu) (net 6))
 (segment (start 94.615 126.365) (end 82.55 114.3) (width 0.762) (layer B.Cu) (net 6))
 (segment (start 94.615 132.08) (end 94.615 126.365) (width 0.762) (layer B.Cu) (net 6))
 (segment (start 97.79 135.255) (end 94.615 132.08) (width 0.762) (layer B.Cu) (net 6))
 (segment (start 102.87 135.255) (end 97.79 135.255) (width 0.762) (layer B.Cu) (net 6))
 (segment (start 105.41 137.795) (end 102.87 135.255) (width 0.762) (layer B.Cu) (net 6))
 (segment (start 110.49 141.605) (end 110.49 137.795) (width 0.762) (layer B.Cu) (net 7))
 (segment (start 78.105 83.82) (end 73.66 83.82) (width 0.762) (layer B.Cu) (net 7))
 (segment (start 85.725 91.44) (end 78.105 83.82) (width 0.762) (layer B.Cu) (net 7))
 (segment (start 85.725 112.395) (end 85.725 91.44) (width 0.762) (layer B.Cu) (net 7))
 (segment (start 94.615 121.285) (end 85.725 112.395) (width 0.762) (layer B.Cu) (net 7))
 (segment (start 102.235 121.285) (end 94.615 121.285) (width 0.762) (layer B.Cu) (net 7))
 (segment (start 106.68 125.73) (end 102.235 121.285) (width 0.762) (layer B.Cu) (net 7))
 (segment (start 106.68 133.985) (end 106.68 125.73) (width 0.762) (layer B.Cu) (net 7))
 (segment (start 110.49 137.795) (end 106.68 133.985) (width 0.762) (layer B.Cu) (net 7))
 (segment (start 115.57 141.605) (end 115.57 138.43) (width 0.762) (layer B.Cu) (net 8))
 (segment (start 84.455 81.28) (end 73.66 81.28) (width 0.762) (layer B.Cu) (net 8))
 (segment (start 88.9 85.725) (end 84.455 81.28) (width 0.762) (layer B.Cu) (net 8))
 (segment (start 88.9 110.49) (end 88.9 85.725) (width 0.762) (layer B.Cu) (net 8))
 (segment (start 95.885 117.475) (end 88.9 110.49) (width 0.762) (layer B.Cu) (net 8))
 (segment (start 111.76 117.475) (end 95.885 117.475) (width 0.762) (layer B.Cu) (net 8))
 (segment (start 117.475 123.19) (end 111.76 117.475) (width 0.762) (layer B.Cu) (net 8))
 (segment (start 117.475 136.525) (end 117.475 123.19) (width 0.762) (layer B.Cu) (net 8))
 (segment (start 115.57 138.43) (end 117.475 136.525) (width 0.762) (layer B.Cu) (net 8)))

